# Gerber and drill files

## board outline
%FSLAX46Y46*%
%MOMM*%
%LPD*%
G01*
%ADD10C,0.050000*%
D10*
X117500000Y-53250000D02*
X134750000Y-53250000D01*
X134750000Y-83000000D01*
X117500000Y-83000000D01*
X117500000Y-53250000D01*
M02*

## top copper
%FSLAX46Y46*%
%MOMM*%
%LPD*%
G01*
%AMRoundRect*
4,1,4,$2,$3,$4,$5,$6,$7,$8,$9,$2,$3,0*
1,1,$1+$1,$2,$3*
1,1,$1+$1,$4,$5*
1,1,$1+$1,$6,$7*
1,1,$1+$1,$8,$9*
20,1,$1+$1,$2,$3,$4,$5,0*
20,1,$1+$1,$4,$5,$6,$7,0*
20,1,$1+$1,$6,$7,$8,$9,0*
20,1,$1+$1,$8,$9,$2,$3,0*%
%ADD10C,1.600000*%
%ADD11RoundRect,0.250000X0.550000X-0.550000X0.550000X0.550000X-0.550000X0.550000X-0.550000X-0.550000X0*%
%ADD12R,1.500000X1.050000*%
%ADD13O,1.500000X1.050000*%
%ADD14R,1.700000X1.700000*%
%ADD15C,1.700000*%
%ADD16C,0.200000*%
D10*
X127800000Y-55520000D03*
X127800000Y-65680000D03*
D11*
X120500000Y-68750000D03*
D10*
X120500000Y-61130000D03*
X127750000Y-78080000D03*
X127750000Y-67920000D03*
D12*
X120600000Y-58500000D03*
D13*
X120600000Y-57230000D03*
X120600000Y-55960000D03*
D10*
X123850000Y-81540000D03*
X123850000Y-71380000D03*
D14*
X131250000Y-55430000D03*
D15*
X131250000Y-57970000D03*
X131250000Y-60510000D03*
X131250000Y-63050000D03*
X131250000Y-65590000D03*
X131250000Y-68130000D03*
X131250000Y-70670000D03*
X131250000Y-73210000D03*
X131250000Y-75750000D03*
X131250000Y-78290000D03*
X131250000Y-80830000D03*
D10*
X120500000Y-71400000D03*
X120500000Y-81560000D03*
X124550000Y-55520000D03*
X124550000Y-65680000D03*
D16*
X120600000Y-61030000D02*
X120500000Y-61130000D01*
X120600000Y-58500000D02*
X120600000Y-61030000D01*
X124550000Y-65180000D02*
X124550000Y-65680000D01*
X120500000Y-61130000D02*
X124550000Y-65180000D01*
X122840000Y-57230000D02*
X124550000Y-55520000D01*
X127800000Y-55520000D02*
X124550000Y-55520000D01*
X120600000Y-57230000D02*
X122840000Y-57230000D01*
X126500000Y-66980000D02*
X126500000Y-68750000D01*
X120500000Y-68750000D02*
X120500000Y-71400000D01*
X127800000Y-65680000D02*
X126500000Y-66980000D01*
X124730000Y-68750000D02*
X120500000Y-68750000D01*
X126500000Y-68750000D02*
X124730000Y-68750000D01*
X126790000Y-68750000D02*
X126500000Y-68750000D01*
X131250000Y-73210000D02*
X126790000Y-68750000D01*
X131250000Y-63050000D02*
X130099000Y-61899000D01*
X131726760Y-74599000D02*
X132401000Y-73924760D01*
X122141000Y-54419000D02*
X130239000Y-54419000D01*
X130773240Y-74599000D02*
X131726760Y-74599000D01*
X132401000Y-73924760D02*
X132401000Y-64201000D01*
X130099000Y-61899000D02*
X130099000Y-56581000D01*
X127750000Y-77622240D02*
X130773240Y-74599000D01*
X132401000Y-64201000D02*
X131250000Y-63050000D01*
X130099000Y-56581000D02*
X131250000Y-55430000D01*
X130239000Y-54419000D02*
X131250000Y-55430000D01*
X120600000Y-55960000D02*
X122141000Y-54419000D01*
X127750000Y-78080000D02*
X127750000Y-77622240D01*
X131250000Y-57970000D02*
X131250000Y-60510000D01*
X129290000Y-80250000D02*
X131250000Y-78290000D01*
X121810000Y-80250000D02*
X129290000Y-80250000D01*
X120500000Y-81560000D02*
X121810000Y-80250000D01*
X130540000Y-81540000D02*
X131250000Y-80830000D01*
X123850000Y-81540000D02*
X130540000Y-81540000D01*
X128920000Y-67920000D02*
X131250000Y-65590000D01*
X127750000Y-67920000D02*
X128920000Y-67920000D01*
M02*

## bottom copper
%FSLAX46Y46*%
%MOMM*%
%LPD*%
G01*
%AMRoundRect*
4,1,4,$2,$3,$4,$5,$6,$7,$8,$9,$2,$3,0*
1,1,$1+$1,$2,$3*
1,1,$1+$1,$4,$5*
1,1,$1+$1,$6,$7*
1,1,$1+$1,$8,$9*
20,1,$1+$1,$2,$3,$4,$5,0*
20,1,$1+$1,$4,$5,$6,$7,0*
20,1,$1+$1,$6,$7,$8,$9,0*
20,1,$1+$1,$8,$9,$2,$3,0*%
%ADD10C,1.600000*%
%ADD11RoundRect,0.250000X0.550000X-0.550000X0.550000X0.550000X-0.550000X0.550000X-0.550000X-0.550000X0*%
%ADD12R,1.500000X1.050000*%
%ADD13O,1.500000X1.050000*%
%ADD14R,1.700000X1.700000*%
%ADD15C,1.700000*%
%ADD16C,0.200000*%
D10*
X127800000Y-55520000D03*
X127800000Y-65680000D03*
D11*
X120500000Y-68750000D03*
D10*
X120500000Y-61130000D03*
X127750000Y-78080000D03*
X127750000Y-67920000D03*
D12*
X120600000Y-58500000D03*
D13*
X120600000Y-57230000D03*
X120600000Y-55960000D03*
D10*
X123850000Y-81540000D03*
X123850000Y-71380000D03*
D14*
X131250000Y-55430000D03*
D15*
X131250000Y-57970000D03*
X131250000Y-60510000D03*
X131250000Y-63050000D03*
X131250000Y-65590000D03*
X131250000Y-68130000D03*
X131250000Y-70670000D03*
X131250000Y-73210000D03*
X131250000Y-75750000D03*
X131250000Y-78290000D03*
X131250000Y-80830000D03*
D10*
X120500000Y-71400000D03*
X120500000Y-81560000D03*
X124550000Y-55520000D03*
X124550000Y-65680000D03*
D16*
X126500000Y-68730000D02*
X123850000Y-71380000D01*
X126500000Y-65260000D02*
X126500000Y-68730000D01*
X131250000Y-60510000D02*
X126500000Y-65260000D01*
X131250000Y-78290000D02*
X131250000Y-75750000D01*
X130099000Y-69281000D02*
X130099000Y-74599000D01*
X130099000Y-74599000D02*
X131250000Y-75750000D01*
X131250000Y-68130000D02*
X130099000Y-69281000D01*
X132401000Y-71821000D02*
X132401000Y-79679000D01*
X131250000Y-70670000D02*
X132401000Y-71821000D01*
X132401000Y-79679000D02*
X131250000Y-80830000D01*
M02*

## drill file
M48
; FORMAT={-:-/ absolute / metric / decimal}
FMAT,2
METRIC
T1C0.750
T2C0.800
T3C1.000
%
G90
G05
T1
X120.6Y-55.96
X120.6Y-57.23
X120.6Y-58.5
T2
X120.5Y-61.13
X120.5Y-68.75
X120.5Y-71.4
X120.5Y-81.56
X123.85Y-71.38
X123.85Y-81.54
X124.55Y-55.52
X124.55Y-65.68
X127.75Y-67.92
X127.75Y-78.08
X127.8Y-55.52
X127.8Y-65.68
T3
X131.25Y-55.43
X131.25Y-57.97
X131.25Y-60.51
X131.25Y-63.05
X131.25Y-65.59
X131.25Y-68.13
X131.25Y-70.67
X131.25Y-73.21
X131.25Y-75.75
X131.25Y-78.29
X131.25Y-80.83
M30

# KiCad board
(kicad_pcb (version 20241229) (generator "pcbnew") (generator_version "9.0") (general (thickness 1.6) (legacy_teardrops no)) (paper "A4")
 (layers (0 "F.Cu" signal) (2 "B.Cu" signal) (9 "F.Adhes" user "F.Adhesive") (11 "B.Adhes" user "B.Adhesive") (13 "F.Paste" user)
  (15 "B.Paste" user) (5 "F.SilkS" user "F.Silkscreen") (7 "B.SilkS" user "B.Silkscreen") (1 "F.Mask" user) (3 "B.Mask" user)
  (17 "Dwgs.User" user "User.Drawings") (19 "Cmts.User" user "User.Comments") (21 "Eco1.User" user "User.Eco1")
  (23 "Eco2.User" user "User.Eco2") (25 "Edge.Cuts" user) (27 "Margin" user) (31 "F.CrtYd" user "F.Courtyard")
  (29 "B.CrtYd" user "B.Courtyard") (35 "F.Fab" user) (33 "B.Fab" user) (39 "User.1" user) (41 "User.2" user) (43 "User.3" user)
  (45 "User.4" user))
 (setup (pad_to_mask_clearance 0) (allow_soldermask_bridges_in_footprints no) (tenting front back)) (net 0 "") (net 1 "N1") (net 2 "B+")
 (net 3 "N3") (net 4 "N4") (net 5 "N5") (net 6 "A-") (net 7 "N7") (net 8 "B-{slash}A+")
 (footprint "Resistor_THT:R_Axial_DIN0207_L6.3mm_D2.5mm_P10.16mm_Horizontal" (layer "F.Cu") (at 127.8 55.52 -90)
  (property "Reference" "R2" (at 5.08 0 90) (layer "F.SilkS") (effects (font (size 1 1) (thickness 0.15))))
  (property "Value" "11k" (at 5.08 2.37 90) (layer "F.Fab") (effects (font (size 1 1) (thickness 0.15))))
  (pad "1" thru_hole circle (at 0 0 270) (size 1.6 1.6) (drill 0.8) (layers "*.Cu" "*.Mask") (remove_unused_layers no) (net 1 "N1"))
  (pad "2" thru_hole circle (at 10.16 0 270) (size 1.6 1.6) (drill 0.8) (layers "*.Cu" "*.Mask") (remove_unused_layers no) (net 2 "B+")))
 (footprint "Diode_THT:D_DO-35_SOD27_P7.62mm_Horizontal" (layer "F.Cu") (at 120.5 68.75 90)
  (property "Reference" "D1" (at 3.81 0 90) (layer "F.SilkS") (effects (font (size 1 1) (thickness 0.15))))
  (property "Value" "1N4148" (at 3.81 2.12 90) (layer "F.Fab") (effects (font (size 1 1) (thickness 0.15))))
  (pad "1" thru_hole roundrect (at 0 0 90) (size 1.6 1.6) (drill 0.8) (layers "*.Cu" "*.Mask") (remove_unused_layers no)
   (roundrect_rratio 0.15625) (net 2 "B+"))
  (pad "2" thru_hole circle (at 7.62 0 90) (size 1.6 1.6) (drill 0.8) (layers "*.Cu" "*.Mask") (remove_unused_layers no) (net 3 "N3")))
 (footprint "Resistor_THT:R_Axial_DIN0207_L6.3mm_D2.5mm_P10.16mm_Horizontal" (layer "F.Cu") (at 127.75 78.08 90)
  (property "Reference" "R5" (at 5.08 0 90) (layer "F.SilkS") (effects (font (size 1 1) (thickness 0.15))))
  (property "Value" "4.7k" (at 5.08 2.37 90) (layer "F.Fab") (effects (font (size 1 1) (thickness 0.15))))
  (pad "1" thru_hole circle (at 0 0 90) (size 1.6 1.6) (drill 0.8) (layers "*.Cu" "*.Mask") (remove_unused_layers no) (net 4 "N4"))
  (pad "2" thru_hole circle (at 10.16 0 90) (size 1.6 1.6) (drill 0.8) (layers "*.Cu" "*.Mask") (remove_unused_layers no) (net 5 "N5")))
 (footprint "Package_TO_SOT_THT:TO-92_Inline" (layer "F.Cu") (at 120.6 58.5 90)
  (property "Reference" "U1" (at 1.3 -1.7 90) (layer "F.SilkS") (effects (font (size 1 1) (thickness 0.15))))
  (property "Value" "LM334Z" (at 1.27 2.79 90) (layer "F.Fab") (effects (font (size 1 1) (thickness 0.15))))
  (pad "1" thru_hole rect (at 0 0 90) (size 1.05 1.5) (drill 0.75) (layers "*.Cu" "*.Mask") (remove_unused_layers no) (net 3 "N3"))
  (pad "2" thru_hole oval (at 1.27 0 90) (size 1.05 1.5) (drill 0.75) (layers "*.Cu" "*.Mask") (remove_unused_layers no) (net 1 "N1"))
  (pad "3" thru_hole oval (at 2.54 0 90) (size 1.05 1.5) (drill 0.75) (layers "*.Cu" "*.Mask") (remove_unused_layers no) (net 4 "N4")))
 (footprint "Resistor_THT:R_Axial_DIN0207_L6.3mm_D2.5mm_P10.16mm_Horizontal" (layer "F.Cu") (at 123.85 81.54 90)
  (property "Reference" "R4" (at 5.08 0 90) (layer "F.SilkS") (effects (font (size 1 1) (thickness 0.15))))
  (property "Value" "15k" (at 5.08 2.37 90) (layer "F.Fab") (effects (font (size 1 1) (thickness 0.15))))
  (pad "1" thru_hole circle (at 0 0 90) (size 1.6 1.6) (drill 0.8) (layers "*.Cu" "*.Mask") (remove_unused_layers no) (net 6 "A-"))
  (pad "2" thru_hole circle (at 10.16 0 90) (size 1.6 1.6) (drill 0.8) (layers "*.Cu" "*.Mask") (remove_unused_layers no) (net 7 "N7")))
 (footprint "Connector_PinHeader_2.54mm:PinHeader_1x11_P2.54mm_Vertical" (layer "F.Cu") (at 131.25 55.43)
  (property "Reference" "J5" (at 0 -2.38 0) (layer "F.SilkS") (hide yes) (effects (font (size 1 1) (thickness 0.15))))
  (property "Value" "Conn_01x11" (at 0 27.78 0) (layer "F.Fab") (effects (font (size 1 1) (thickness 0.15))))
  (pad "1" thru_hole rect (at 0 0) (size 1.7 1.7) (drill 1) (layers "*.Cu" "*.Mask") (remove_unused_layers no) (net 4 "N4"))
  (pad "2" thru_hole circle (at 0 2.54) (size 1.7 1.7) (drill 1) (layers "*.Cu" "*.Mask") (remove_unused_layers no) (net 7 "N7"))
  (pad "3" thru_hole circle (at 0 5.08) (size 1.7 1.7) (drill 1) (layers "*.Cu" "*.Mask") (remove_unused_layers no) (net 7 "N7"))
  (pad "4" thru_hole circle (at 0 7.62) (size 1.7 1.7) (drill 1) (layers "*.Cu" "*.Mask") (remove_unused_layers no) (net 4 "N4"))
  (pad "5" thru_hole circle (at 0 10.16) (size 1.7 1.7) (drill 1) (layers "*.Cu" "*.Mask") (remove_unused_layers no) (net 5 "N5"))
  (pad "6" thru_hole circle (at 0 12.7) (size 1.7 1.7) (drill 1) (layers "*.Cu" "*.Mask") (remove_unused_layers no) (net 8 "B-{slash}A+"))
  (pad "7" thru_hole circle (at 0 15.24) (size 1.7 1.7) (drill 1) (layers "*.Cu" "*.Mask") (remove_unused_layers no) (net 6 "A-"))
  (pad "8" thru_hole circle (at 0 17.78) (size 1.7 1.7) (drill 1) (layers "*.Cu" "*.Mask") (remove_unused_layers no) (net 2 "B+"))
  (pad "9" thru_hole circle (at 0 20.32) (size 1.7 1.7) (drill 1) (layers "*.Cu" "*.Mask") (remove_unused_layers no) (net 8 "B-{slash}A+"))
  (pad "10" thru_hole circle (at 0 22.86) (size 1.7 1.7) (drill 1) (layers "*.Cu" "*.Mask") (remove_unused_layers no) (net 8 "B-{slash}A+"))
  (pad "11" thru_hole circle (at 0 25.4) (size 1.7 1.7) (drill 1) (layers "*.Cu" "*.Mask") (remove_unused_layers no) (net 6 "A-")))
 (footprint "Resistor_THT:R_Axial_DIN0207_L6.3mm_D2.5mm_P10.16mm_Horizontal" (layer "F.Cu") (at 120.5 71.4 -90)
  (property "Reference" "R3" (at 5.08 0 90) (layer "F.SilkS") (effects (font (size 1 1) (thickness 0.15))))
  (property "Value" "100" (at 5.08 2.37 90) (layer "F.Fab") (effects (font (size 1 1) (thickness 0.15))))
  (pad "1" thru_hole circle (at 0 0 270) (size 1.6 1.6) (drill 0.8) (layers "*.Cu" "*.Mask") (remove_unused_layers no) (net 2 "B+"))
  (pad "2" thru_hole circle (at 10.16 0 270) (size 1.6 1.6) (drill 0.8) (layers "*.Cu" "*.Mask") (remove_unused_layers no)
   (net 8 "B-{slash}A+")))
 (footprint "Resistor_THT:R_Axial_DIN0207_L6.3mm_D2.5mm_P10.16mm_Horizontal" (layer "F.Cu") (at 124.55 55.52 -90)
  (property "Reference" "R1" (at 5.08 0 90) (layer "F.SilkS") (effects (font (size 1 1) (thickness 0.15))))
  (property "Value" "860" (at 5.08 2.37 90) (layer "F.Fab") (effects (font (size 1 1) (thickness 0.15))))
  (pad "1" thru_hole circle (at 0 0 270) (size 1.6 1.6) (drill 0.8) (layers "*.Cu" "*.Mask") (remove_unused_layers no) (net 1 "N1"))
  (pad "2" thru_hole circle (at 10.16 0 270) (size 1.6 1.6) (drill 0.8) (layers "*.Cu" "*.Mask") (remove_unused_layers no) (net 3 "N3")))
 (gr_rect (start 117.5 53.25) (end 134.75 83) (stroke (width 0.05) (type default)) (fill no) (layer "Edge.Cuts"))
 (segment (start 120.6 61.03) (end 120.5 61.13) (width 0.2) (layer "F.Cu") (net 3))
 (segment (start 120.6 58.5) (end 120.6 61.03) (width 0.2) (layer "F.Cu") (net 3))
 (segment (start 124.55 65.18) (end 124.55 65.68) (width 0.2) (layer "F.Cu") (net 3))
 (segment (start 120.5 61.13) (end 124.55 65.18) (width 0.2) (layer "F.Cu") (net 3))
 (segment (start 122.84 57.23) (end 124.55 55.52) (width 0.2) (layer "F.Cu") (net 1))
 (segment (start 127.8 55.52) (end 124.55 55.52) (width 0.2) (layer "F.Cu") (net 1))
 (segment (start 120.6 57.23) (end 122.84 57.23) (width 0.2) (layer "F.Cu") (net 1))
 (segment (start 126.5 66.98) (end 126.5 68.75) (width 0.2) (layer "F.Cu") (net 2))
 (segment (start 120.5 68.75) (end 120.5 71.4) (width 0.2) (layer "F.Cu") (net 2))
 (segment (start 127.8 65.68) (end 126.5 66.98) (width 0.2) (layer "F.Cu") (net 2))
 (segment (start 124.73 68.75) (end 120.5 68.75) (width 0.2) (layer "F.Cu") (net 2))
 (segment (start 126.5 68.75) (end 124.73 68.75) (width 0.2) (layer "F.Cu") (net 2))
 (segment (start 126.79 68.75) (end 126.5 68.75) (width 0.2) (layer "F.Cu") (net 2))
 (segment (start 131.25 73.21) (end 126.79 68.75) (width 0.2) (layer "F.Cu") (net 2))
 (segment (start 131.25 63.05) (end 130.099 61.899) (width 0.2) (layer "F.Cu") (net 4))
 (segment (start 131.72676 74.599) (end 132.401 73.92476) (width 0.2) (layer "F.Cu") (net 4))
 (segment (start 122.141 54.419) (end 130.239 54.419) (width 0.2) (layer "F.Cu") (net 4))
 (segment (start 130.77324 74.599) (end 131.72676 74.599) (width 0.2) (layer "F.Cu") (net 4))
 (segment (start 132.401 73.92476) (end 132.401 64.201) (width 0.2) (layer "F.Cu") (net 4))
 (segment (start 130.099 61.899) (end 130.099 56.581) (width 0.2) (layer "F.Cu") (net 4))
 (segment (start 127.75 77.62224) (end 130.77324 74.599) (width 0.2) (layer "F.Cu") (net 4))
 (segment (start 132.401 64.201) (end 131.25 63.05) (width 0.2) (layer "F.Cu") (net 4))
 (segment (start 130.099 56.581) (end 131.25 55.43) (width 0.2) (layer "F.Cu") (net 4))
 (segment (start 130.239 54.419) (end 131.25 55.43) (width 0.2) (layer "F.Cu") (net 4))
 (segment (start 120.6 55.96) (end 122.141 54.419) (width 0.2) (layer "F.Cu") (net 4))
 (segment (start 127.75 78.08) (end 127.75 77.62224) (width 0.2) (layer "F.Cu") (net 4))
 (segment (start 131.25 57.97) (end 131.25 60.51) (width 0.2) (layer "F.Cu") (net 7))
 (segment (start 126.5 68.73) (end 123.85 71.38) (width 0.2) (layer "B.Cu") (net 7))
 (segment (start 126.5 65.26) (end 126.5 68.73) (width 0.2) (layer "B.Cu") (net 7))
 (segment (start 131.25 60.51) (end 126.5 65.26) (width 0.2) (layer "B.Cu") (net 7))
 (segment (start 129.29 80.25) (end 131.25 78.29) (width 0.2) (layer "F.Cu") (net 8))
 (segment (start 121.81 80.25) (end 129.29 80.25) (width 0.2) (layer "F.Cu") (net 8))
 (segment (start 120.5 81.56) (end 121.81 80.25) (width 0.2) (layer "F.Cu") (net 8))
 (segment (start 131.25 78.29) (end 131.25 75.75) (width 0.2) (layer "B.Cu") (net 8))
 (segment (start 130.099 69.281) (end 130.099 74.599) (width 0.2) (layer "B.Cu") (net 8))
 (segment (start 130.099 74.599) (end 131.25 75.75) (width 0.2) (layer "B.Cu") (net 8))
 (segment (start 131.25 68.13) (end 130.099 69.281) (width 0.2) (layer "B.Cu") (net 8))
 (segment (start 130.54 81.54) (end 131.25 80.83) (width 0.2) (layer "F.Cu") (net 6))
 (segment (start 123.85 81.54) (end 130.54 81.54) (width 0.2) (layer "F.Cu") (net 6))
 (segment (start 132.401 71.821) (end 132.401 79.679) (width 0.2) (layer "B.Cu") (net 6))
 (segment (start 131.25 70.67) (end 132.401 71.821) (width 0.2) (layer "B.Cu") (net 6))
 (segment (start 132.401 79.679) (end 131.25 80.83) (width 0.2) (layer "B.Cu") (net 6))
 (segment (start 128.92 67.92) (end 131.25 65.59) (width 0.2) (layer "F.Cu") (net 5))
 (segment (start 127.75 67.92) (end 128.92 67.92) (width 0.2) (layer "F.Cu") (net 5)))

